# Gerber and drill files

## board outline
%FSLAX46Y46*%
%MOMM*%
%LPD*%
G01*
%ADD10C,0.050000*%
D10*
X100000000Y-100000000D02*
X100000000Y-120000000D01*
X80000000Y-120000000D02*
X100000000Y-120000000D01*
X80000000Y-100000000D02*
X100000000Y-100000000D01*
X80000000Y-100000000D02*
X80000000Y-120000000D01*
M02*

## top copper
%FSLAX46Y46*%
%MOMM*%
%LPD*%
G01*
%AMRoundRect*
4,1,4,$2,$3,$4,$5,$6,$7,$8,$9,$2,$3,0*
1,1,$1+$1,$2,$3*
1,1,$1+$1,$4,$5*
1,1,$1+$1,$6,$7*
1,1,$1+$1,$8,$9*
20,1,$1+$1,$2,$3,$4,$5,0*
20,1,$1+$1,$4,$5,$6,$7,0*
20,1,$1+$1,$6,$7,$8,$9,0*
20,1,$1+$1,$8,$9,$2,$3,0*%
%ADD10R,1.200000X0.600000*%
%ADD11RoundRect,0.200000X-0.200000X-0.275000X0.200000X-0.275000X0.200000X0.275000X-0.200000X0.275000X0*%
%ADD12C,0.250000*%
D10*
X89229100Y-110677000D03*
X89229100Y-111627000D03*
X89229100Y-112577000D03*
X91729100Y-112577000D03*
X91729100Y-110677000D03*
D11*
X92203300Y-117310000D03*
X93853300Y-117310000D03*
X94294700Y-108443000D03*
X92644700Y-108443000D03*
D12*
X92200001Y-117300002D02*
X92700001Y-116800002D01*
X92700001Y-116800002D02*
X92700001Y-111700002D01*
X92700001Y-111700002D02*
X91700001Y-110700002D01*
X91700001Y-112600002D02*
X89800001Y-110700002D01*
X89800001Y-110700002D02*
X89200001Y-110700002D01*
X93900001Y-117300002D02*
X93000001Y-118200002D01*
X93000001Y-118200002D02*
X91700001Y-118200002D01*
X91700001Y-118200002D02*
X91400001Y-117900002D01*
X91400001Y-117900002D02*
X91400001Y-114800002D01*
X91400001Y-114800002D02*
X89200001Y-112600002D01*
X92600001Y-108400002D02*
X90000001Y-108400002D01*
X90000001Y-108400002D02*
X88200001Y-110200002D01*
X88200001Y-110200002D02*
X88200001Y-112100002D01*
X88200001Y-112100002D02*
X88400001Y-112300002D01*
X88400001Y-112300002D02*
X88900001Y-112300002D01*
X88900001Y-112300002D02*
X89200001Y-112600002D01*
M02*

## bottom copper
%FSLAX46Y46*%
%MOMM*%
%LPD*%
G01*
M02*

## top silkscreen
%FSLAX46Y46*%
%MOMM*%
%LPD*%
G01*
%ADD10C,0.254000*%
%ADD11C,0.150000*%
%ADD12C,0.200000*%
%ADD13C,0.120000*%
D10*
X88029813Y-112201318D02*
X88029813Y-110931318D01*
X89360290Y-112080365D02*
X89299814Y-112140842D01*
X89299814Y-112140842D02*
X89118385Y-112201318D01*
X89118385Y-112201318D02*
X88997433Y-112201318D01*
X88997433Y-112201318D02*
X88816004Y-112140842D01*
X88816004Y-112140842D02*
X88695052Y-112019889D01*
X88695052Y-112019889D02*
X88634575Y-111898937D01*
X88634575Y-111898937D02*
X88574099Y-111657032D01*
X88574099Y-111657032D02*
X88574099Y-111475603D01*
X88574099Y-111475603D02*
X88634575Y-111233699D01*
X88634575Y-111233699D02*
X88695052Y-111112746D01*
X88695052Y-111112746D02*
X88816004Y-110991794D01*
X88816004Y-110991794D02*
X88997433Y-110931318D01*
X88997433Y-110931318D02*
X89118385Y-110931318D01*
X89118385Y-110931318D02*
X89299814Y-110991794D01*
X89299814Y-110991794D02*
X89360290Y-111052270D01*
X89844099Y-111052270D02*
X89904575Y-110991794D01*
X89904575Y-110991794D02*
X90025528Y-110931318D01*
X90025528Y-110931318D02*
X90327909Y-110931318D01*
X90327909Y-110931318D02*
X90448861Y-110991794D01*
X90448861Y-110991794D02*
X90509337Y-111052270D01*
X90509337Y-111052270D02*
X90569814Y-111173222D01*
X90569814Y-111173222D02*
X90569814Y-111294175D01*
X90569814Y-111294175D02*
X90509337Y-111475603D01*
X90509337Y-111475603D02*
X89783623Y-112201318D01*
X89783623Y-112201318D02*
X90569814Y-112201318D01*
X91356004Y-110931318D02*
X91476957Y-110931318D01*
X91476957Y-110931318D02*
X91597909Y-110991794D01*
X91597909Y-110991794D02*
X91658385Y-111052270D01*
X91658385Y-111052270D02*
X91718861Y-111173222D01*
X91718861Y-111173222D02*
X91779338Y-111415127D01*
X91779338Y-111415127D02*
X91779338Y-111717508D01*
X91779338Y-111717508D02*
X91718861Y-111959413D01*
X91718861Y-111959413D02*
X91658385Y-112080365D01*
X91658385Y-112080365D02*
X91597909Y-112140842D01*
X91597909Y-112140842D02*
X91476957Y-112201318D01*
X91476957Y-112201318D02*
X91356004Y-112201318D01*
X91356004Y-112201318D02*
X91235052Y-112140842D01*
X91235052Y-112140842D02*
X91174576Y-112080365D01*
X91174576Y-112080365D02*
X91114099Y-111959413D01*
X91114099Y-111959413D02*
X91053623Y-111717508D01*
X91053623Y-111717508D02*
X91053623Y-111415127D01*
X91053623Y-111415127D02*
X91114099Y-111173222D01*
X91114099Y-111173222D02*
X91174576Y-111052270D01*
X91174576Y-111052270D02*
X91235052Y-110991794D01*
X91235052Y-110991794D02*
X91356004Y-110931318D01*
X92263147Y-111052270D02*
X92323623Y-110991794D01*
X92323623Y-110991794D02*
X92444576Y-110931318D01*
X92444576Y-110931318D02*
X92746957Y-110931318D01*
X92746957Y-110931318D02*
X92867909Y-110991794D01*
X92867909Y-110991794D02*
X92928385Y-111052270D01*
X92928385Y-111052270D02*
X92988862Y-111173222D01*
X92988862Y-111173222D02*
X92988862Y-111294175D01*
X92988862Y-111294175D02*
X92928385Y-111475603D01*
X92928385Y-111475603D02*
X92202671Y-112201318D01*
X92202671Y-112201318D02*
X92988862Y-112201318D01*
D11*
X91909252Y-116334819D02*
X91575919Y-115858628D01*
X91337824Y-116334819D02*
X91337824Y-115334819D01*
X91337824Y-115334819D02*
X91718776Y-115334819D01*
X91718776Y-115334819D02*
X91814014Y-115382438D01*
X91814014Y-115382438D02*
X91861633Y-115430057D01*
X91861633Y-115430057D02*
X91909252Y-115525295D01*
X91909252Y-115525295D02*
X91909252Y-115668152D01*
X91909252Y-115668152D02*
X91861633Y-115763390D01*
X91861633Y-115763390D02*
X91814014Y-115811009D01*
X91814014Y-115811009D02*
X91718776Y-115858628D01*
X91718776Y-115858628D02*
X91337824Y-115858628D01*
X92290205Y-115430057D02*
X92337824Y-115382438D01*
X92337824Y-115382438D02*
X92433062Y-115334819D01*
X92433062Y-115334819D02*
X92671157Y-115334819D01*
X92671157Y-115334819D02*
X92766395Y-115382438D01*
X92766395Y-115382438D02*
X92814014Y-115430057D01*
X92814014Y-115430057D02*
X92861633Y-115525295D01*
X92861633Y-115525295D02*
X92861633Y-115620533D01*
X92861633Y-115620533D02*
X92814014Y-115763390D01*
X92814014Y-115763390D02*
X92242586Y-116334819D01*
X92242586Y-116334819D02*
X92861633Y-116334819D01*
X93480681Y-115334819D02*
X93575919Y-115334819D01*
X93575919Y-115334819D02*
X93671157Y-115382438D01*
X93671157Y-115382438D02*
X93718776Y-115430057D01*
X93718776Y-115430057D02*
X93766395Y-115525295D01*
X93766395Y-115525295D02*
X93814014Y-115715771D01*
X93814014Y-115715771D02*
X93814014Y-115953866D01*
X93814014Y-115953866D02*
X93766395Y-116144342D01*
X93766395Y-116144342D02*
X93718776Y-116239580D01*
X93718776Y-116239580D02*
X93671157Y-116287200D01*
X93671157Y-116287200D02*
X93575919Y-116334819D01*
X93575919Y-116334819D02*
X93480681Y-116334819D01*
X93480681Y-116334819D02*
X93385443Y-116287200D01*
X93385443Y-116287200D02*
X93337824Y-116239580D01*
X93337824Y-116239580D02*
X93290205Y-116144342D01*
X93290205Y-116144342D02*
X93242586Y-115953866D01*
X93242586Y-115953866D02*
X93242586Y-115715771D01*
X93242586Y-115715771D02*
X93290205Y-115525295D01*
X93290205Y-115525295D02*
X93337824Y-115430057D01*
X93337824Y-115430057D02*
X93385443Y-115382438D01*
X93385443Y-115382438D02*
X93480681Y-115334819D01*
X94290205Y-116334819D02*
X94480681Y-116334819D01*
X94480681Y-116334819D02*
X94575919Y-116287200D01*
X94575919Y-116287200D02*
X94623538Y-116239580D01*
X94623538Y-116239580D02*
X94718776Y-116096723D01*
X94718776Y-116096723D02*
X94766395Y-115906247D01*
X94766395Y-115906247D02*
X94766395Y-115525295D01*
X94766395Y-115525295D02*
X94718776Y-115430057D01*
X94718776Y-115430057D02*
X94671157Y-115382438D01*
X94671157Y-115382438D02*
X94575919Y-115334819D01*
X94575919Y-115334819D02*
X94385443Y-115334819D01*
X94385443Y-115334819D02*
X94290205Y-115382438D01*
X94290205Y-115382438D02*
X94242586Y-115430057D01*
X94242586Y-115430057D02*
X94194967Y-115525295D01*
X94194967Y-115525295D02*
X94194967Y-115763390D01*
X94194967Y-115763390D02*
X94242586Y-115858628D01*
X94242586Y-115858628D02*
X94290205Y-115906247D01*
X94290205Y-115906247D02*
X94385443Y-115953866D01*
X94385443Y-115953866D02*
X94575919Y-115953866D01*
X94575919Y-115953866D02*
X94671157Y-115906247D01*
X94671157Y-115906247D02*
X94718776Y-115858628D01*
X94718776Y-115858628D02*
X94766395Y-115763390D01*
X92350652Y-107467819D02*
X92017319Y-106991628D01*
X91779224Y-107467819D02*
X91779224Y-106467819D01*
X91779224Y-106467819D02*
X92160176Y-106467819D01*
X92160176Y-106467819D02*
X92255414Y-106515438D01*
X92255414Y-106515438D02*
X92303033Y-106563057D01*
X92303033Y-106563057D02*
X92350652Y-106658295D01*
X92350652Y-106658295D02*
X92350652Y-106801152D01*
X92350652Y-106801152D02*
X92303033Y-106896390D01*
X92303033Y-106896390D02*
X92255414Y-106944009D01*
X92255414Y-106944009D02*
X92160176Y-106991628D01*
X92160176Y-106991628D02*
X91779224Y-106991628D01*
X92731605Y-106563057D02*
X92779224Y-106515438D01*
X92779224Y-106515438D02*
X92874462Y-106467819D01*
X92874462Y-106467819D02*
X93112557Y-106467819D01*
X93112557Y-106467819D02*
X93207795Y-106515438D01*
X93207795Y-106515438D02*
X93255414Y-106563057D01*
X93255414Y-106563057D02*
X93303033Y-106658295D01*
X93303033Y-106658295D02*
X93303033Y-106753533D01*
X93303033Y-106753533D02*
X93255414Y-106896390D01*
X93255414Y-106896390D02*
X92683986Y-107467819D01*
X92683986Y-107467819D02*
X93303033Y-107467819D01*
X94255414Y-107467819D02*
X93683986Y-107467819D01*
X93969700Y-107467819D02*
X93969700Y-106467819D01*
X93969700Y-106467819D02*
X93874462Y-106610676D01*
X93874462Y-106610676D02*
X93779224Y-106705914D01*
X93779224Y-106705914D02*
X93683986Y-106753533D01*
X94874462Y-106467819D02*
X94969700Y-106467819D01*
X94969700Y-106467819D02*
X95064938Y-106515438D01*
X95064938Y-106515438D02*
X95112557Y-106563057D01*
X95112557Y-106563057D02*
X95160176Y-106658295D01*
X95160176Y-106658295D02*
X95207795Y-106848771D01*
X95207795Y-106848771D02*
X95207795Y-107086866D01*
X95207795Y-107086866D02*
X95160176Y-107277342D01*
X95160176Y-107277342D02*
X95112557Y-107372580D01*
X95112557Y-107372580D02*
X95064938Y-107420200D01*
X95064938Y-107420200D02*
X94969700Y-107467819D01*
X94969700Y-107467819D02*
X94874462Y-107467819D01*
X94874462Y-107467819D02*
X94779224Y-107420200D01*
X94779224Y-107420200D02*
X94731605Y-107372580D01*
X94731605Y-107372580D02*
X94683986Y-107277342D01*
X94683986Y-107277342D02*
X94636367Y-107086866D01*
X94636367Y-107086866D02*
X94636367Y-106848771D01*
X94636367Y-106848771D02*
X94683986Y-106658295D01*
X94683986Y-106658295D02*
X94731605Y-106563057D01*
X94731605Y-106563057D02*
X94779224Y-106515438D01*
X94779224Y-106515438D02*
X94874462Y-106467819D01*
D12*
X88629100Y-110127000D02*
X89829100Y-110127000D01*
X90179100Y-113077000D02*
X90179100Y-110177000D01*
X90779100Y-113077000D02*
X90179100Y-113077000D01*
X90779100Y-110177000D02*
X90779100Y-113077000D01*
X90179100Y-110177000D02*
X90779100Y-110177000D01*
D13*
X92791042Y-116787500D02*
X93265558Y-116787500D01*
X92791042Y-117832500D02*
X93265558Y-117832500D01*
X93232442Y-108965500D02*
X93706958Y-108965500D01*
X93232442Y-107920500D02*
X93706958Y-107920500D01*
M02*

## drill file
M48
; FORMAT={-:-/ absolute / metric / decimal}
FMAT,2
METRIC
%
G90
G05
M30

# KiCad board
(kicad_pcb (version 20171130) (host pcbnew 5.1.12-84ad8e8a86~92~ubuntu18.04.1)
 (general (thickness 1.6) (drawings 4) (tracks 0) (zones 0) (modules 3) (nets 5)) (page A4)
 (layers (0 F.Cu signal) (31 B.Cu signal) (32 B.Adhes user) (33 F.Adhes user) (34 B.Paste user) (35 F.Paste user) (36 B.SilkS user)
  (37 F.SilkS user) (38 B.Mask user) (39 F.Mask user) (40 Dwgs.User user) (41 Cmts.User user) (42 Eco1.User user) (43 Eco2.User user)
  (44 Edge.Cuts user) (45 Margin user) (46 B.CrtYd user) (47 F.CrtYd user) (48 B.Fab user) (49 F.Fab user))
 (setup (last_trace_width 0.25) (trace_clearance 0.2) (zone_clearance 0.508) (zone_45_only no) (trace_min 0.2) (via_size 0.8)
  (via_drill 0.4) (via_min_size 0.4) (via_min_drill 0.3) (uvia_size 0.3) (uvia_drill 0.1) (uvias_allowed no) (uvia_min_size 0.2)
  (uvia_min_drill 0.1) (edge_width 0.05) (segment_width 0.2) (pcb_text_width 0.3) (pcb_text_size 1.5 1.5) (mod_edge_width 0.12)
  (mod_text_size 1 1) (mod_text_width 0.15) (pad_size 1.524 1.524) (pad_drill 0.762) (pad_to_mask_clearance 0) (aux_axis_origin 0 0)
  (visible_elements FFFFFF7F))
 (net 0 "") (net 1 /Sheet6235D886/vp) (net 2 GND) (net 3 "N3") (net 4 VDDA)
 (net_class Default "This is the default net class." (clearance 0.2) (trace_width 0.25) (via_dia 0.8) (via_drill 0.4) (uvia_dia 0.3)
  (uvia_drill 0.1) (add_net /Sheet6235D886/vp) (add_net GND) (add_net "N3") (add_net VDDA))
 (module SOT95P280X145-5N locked (layer F.Cu) (at 90.479100 111.627000)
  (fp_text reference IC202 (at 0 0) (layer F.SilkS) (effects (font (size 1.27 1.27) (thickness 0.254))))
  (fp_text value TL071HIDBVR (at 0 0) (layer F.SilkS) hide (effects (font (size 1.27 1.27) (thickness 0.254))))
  (fp_line (start -1.85 -1.5) (end -0.65 -1.5) (layer F.SilkS) (width 0.2))
  (fp_line (start -0.3 1.45) (end -0.3 -1.45) (layer F.SilkS) (width 0.2))
  (fp_line (start 0.3 1.45) (end -0.3 1.45) (layer F.SilkS) (width 0.2))
  (fp_line (start 0.3 -1.45) (end 0.3 1.45) (layer F.SilkS) (width 0.2))
  (fp_line (start -0.3 -1.45) (end 0.3 -1.45) (layer F.SilkS) (width 0.2))
  (pad 1 smd rect (at -1.25 -0.95 90.000000) (size 0.6 1.2) (layers F.Cu F.Mask F.Paste) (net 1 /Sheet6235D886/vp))
  (pad 2 smd rect (at -1.25 0 90.000000) (size 0.6 1.2) (layers F.Cu F.Mask F.Paste) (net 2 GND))
  (pad 3 smd rect (at -1.25 0.95 90.000000) (size 0.6 1.2) (layers F.Cu F.Mask F.Paste) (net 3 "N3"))
  (pad 4 smd rect (at 1.25 0.95 90.000000) (size 0.6 1.2) (layers F.Cu F.Mask F.Paste) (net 1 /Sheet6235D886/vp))
  (pad 5 smd rect (at 1.25 -0.95 90.000000) (size 0.6 1.2) (layers F.Cu F.Mask F.Paste) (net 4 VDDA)))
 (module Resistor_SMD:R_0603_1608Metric (layer F.Cu) (at 93.028300 117.310000)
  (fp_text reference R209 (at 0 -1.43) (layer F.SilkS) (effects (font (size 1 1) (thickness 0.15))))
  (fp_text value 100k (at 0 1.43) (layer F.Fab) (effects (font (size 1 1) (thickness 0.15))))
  (fp_line (start -0.237258 -0.5225) (end 0.237258 -0.5225) (layer F.SilkS) (width 0.12))
  (fp_line (start -0.237258 0.5225) (end 0.237258 0.5225) (layer F.SilkS) (width 0.12))
  (pad 1 smd roundrect (at -0.825 0) (size 0.8 0.95) (layers F.Cu F.Mask F.Paste) (roundrect_rratio 0.25) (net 4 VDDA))
  (pad 2 smd roundrect (at 0.825 0) (size 0.8 0.95) (layers F.Cu F.Mask F.Paste) (roundrect_rratio 0.25) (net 3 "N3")))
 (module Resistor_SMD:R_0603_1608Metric (layer F.Cu) (at 93.469700 108.443000)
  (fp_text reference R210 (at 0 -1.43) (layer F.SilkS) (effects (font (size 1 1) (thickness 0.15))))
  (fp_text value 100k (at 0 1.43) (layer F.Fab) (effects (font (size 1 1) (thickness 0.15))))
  (fp_line (start -0.237258 0.5225) (end 0.237258 0.5225) (layer F.SilkS) (width 0.12))
  (fp_line (start -0.237258 -0.5225) (end 0.237258 -0.5225) (layer F.SilkS) (width 0.12))
  (pad 2 smd roundrect (at 0.825 0) (size 0.8 0.95) (layers F.Cu F.Mask F.Paste) (roundrect_rratio 0.25) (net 2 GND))
  (pad 1 smd roundrect (at -0.825 0) (size 0.8 0.95) (layers F.Cu F.Mask F.Paste) (roundrect_rratio 0.25) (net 3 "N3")))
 (gr_line (start 100 100) (end 100 120) (layer Edge.Cuts) (width 0.05))
 (gr_line (start 80 120) (end 100 120) (layer Edge.Cuts) (width 0.05))
 (gr_line (start 80 100) (end 100 100) (layer Edge.Cuts) (width 0.05))
 (gr_line (start 80 100) (end 80 120) (layer Edge.Cuts) (width 0.05))
 (segment (start 92.200001 117.300002) (end 92.700001 116.800002) (width 0.250000) (layer F.Cu) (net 4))
 (segment (start 92.700001 116.800002) (end 92.700001 111.700002) (width 0.250000) (layer F.Cu) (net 4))
 (segment (start 92.700001 111.700002) (end 91.700001 110.700002) (width 0.250000) (layer F.Cu) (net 4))
 (segment (start 91.700001 112.600002) (end 89.800001 110.700002) (width 0.250000) (layer F.Cu) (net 1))
 (segment (start 89.800001 110.700002) (end 89.200001 110.700002) (width 0.250000) (layer F.Cu) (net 1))
 (segment (start 93.900001 117.300002) (end 93.000001 118.200002) (width 0.250000) (layer F.Cu) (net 3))
 (segment (start 93.000001 118.200002) (end 91.700001 118.200002) (width 0.250000) (layer F.Cu) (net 3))
 (segment (start 91.700001 118.200002) (end 91.400001 117.900002) (width 0.250000) (layer F.Cu) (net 3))
 (segment (start 91.400001 117.900002) (end 91.400001 114.800002) (width 0.250000) (layer F.Cu) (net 3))
 (segment (start 91.400001 114.800002) (end 89.200001 112.600002) (width 0.250000) (layer F.Cu) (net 3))
 (segment (start 92.600001 108.400002) (end 90.000001 108.400002) (width 0.250000) (layer F.Cu) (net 3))
 (segment (start 90.000001 108.400002) (end 88.200001 110.200002) (width 0.250000) (layer F.Cu) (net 3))
 (segment (start 88.200001 110.200002) (end 88.200001 112.100002) (width 0.250000) (layer F.Cu) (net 3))
 (segment (start 88.200001 112.100002) (end 88.400001 112.300002) (width 0.250000) (layer F.Cu) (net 3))
 (segment (start 88.400001 112.300002) (end 88.900001 112.300002) (width 0.250000) (layer F.Cu) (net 3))
 (segment (start 88.900001 112.300002) (end 89.200001 112.600002) (width 0.250000) (layer F.Cu) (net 3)))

